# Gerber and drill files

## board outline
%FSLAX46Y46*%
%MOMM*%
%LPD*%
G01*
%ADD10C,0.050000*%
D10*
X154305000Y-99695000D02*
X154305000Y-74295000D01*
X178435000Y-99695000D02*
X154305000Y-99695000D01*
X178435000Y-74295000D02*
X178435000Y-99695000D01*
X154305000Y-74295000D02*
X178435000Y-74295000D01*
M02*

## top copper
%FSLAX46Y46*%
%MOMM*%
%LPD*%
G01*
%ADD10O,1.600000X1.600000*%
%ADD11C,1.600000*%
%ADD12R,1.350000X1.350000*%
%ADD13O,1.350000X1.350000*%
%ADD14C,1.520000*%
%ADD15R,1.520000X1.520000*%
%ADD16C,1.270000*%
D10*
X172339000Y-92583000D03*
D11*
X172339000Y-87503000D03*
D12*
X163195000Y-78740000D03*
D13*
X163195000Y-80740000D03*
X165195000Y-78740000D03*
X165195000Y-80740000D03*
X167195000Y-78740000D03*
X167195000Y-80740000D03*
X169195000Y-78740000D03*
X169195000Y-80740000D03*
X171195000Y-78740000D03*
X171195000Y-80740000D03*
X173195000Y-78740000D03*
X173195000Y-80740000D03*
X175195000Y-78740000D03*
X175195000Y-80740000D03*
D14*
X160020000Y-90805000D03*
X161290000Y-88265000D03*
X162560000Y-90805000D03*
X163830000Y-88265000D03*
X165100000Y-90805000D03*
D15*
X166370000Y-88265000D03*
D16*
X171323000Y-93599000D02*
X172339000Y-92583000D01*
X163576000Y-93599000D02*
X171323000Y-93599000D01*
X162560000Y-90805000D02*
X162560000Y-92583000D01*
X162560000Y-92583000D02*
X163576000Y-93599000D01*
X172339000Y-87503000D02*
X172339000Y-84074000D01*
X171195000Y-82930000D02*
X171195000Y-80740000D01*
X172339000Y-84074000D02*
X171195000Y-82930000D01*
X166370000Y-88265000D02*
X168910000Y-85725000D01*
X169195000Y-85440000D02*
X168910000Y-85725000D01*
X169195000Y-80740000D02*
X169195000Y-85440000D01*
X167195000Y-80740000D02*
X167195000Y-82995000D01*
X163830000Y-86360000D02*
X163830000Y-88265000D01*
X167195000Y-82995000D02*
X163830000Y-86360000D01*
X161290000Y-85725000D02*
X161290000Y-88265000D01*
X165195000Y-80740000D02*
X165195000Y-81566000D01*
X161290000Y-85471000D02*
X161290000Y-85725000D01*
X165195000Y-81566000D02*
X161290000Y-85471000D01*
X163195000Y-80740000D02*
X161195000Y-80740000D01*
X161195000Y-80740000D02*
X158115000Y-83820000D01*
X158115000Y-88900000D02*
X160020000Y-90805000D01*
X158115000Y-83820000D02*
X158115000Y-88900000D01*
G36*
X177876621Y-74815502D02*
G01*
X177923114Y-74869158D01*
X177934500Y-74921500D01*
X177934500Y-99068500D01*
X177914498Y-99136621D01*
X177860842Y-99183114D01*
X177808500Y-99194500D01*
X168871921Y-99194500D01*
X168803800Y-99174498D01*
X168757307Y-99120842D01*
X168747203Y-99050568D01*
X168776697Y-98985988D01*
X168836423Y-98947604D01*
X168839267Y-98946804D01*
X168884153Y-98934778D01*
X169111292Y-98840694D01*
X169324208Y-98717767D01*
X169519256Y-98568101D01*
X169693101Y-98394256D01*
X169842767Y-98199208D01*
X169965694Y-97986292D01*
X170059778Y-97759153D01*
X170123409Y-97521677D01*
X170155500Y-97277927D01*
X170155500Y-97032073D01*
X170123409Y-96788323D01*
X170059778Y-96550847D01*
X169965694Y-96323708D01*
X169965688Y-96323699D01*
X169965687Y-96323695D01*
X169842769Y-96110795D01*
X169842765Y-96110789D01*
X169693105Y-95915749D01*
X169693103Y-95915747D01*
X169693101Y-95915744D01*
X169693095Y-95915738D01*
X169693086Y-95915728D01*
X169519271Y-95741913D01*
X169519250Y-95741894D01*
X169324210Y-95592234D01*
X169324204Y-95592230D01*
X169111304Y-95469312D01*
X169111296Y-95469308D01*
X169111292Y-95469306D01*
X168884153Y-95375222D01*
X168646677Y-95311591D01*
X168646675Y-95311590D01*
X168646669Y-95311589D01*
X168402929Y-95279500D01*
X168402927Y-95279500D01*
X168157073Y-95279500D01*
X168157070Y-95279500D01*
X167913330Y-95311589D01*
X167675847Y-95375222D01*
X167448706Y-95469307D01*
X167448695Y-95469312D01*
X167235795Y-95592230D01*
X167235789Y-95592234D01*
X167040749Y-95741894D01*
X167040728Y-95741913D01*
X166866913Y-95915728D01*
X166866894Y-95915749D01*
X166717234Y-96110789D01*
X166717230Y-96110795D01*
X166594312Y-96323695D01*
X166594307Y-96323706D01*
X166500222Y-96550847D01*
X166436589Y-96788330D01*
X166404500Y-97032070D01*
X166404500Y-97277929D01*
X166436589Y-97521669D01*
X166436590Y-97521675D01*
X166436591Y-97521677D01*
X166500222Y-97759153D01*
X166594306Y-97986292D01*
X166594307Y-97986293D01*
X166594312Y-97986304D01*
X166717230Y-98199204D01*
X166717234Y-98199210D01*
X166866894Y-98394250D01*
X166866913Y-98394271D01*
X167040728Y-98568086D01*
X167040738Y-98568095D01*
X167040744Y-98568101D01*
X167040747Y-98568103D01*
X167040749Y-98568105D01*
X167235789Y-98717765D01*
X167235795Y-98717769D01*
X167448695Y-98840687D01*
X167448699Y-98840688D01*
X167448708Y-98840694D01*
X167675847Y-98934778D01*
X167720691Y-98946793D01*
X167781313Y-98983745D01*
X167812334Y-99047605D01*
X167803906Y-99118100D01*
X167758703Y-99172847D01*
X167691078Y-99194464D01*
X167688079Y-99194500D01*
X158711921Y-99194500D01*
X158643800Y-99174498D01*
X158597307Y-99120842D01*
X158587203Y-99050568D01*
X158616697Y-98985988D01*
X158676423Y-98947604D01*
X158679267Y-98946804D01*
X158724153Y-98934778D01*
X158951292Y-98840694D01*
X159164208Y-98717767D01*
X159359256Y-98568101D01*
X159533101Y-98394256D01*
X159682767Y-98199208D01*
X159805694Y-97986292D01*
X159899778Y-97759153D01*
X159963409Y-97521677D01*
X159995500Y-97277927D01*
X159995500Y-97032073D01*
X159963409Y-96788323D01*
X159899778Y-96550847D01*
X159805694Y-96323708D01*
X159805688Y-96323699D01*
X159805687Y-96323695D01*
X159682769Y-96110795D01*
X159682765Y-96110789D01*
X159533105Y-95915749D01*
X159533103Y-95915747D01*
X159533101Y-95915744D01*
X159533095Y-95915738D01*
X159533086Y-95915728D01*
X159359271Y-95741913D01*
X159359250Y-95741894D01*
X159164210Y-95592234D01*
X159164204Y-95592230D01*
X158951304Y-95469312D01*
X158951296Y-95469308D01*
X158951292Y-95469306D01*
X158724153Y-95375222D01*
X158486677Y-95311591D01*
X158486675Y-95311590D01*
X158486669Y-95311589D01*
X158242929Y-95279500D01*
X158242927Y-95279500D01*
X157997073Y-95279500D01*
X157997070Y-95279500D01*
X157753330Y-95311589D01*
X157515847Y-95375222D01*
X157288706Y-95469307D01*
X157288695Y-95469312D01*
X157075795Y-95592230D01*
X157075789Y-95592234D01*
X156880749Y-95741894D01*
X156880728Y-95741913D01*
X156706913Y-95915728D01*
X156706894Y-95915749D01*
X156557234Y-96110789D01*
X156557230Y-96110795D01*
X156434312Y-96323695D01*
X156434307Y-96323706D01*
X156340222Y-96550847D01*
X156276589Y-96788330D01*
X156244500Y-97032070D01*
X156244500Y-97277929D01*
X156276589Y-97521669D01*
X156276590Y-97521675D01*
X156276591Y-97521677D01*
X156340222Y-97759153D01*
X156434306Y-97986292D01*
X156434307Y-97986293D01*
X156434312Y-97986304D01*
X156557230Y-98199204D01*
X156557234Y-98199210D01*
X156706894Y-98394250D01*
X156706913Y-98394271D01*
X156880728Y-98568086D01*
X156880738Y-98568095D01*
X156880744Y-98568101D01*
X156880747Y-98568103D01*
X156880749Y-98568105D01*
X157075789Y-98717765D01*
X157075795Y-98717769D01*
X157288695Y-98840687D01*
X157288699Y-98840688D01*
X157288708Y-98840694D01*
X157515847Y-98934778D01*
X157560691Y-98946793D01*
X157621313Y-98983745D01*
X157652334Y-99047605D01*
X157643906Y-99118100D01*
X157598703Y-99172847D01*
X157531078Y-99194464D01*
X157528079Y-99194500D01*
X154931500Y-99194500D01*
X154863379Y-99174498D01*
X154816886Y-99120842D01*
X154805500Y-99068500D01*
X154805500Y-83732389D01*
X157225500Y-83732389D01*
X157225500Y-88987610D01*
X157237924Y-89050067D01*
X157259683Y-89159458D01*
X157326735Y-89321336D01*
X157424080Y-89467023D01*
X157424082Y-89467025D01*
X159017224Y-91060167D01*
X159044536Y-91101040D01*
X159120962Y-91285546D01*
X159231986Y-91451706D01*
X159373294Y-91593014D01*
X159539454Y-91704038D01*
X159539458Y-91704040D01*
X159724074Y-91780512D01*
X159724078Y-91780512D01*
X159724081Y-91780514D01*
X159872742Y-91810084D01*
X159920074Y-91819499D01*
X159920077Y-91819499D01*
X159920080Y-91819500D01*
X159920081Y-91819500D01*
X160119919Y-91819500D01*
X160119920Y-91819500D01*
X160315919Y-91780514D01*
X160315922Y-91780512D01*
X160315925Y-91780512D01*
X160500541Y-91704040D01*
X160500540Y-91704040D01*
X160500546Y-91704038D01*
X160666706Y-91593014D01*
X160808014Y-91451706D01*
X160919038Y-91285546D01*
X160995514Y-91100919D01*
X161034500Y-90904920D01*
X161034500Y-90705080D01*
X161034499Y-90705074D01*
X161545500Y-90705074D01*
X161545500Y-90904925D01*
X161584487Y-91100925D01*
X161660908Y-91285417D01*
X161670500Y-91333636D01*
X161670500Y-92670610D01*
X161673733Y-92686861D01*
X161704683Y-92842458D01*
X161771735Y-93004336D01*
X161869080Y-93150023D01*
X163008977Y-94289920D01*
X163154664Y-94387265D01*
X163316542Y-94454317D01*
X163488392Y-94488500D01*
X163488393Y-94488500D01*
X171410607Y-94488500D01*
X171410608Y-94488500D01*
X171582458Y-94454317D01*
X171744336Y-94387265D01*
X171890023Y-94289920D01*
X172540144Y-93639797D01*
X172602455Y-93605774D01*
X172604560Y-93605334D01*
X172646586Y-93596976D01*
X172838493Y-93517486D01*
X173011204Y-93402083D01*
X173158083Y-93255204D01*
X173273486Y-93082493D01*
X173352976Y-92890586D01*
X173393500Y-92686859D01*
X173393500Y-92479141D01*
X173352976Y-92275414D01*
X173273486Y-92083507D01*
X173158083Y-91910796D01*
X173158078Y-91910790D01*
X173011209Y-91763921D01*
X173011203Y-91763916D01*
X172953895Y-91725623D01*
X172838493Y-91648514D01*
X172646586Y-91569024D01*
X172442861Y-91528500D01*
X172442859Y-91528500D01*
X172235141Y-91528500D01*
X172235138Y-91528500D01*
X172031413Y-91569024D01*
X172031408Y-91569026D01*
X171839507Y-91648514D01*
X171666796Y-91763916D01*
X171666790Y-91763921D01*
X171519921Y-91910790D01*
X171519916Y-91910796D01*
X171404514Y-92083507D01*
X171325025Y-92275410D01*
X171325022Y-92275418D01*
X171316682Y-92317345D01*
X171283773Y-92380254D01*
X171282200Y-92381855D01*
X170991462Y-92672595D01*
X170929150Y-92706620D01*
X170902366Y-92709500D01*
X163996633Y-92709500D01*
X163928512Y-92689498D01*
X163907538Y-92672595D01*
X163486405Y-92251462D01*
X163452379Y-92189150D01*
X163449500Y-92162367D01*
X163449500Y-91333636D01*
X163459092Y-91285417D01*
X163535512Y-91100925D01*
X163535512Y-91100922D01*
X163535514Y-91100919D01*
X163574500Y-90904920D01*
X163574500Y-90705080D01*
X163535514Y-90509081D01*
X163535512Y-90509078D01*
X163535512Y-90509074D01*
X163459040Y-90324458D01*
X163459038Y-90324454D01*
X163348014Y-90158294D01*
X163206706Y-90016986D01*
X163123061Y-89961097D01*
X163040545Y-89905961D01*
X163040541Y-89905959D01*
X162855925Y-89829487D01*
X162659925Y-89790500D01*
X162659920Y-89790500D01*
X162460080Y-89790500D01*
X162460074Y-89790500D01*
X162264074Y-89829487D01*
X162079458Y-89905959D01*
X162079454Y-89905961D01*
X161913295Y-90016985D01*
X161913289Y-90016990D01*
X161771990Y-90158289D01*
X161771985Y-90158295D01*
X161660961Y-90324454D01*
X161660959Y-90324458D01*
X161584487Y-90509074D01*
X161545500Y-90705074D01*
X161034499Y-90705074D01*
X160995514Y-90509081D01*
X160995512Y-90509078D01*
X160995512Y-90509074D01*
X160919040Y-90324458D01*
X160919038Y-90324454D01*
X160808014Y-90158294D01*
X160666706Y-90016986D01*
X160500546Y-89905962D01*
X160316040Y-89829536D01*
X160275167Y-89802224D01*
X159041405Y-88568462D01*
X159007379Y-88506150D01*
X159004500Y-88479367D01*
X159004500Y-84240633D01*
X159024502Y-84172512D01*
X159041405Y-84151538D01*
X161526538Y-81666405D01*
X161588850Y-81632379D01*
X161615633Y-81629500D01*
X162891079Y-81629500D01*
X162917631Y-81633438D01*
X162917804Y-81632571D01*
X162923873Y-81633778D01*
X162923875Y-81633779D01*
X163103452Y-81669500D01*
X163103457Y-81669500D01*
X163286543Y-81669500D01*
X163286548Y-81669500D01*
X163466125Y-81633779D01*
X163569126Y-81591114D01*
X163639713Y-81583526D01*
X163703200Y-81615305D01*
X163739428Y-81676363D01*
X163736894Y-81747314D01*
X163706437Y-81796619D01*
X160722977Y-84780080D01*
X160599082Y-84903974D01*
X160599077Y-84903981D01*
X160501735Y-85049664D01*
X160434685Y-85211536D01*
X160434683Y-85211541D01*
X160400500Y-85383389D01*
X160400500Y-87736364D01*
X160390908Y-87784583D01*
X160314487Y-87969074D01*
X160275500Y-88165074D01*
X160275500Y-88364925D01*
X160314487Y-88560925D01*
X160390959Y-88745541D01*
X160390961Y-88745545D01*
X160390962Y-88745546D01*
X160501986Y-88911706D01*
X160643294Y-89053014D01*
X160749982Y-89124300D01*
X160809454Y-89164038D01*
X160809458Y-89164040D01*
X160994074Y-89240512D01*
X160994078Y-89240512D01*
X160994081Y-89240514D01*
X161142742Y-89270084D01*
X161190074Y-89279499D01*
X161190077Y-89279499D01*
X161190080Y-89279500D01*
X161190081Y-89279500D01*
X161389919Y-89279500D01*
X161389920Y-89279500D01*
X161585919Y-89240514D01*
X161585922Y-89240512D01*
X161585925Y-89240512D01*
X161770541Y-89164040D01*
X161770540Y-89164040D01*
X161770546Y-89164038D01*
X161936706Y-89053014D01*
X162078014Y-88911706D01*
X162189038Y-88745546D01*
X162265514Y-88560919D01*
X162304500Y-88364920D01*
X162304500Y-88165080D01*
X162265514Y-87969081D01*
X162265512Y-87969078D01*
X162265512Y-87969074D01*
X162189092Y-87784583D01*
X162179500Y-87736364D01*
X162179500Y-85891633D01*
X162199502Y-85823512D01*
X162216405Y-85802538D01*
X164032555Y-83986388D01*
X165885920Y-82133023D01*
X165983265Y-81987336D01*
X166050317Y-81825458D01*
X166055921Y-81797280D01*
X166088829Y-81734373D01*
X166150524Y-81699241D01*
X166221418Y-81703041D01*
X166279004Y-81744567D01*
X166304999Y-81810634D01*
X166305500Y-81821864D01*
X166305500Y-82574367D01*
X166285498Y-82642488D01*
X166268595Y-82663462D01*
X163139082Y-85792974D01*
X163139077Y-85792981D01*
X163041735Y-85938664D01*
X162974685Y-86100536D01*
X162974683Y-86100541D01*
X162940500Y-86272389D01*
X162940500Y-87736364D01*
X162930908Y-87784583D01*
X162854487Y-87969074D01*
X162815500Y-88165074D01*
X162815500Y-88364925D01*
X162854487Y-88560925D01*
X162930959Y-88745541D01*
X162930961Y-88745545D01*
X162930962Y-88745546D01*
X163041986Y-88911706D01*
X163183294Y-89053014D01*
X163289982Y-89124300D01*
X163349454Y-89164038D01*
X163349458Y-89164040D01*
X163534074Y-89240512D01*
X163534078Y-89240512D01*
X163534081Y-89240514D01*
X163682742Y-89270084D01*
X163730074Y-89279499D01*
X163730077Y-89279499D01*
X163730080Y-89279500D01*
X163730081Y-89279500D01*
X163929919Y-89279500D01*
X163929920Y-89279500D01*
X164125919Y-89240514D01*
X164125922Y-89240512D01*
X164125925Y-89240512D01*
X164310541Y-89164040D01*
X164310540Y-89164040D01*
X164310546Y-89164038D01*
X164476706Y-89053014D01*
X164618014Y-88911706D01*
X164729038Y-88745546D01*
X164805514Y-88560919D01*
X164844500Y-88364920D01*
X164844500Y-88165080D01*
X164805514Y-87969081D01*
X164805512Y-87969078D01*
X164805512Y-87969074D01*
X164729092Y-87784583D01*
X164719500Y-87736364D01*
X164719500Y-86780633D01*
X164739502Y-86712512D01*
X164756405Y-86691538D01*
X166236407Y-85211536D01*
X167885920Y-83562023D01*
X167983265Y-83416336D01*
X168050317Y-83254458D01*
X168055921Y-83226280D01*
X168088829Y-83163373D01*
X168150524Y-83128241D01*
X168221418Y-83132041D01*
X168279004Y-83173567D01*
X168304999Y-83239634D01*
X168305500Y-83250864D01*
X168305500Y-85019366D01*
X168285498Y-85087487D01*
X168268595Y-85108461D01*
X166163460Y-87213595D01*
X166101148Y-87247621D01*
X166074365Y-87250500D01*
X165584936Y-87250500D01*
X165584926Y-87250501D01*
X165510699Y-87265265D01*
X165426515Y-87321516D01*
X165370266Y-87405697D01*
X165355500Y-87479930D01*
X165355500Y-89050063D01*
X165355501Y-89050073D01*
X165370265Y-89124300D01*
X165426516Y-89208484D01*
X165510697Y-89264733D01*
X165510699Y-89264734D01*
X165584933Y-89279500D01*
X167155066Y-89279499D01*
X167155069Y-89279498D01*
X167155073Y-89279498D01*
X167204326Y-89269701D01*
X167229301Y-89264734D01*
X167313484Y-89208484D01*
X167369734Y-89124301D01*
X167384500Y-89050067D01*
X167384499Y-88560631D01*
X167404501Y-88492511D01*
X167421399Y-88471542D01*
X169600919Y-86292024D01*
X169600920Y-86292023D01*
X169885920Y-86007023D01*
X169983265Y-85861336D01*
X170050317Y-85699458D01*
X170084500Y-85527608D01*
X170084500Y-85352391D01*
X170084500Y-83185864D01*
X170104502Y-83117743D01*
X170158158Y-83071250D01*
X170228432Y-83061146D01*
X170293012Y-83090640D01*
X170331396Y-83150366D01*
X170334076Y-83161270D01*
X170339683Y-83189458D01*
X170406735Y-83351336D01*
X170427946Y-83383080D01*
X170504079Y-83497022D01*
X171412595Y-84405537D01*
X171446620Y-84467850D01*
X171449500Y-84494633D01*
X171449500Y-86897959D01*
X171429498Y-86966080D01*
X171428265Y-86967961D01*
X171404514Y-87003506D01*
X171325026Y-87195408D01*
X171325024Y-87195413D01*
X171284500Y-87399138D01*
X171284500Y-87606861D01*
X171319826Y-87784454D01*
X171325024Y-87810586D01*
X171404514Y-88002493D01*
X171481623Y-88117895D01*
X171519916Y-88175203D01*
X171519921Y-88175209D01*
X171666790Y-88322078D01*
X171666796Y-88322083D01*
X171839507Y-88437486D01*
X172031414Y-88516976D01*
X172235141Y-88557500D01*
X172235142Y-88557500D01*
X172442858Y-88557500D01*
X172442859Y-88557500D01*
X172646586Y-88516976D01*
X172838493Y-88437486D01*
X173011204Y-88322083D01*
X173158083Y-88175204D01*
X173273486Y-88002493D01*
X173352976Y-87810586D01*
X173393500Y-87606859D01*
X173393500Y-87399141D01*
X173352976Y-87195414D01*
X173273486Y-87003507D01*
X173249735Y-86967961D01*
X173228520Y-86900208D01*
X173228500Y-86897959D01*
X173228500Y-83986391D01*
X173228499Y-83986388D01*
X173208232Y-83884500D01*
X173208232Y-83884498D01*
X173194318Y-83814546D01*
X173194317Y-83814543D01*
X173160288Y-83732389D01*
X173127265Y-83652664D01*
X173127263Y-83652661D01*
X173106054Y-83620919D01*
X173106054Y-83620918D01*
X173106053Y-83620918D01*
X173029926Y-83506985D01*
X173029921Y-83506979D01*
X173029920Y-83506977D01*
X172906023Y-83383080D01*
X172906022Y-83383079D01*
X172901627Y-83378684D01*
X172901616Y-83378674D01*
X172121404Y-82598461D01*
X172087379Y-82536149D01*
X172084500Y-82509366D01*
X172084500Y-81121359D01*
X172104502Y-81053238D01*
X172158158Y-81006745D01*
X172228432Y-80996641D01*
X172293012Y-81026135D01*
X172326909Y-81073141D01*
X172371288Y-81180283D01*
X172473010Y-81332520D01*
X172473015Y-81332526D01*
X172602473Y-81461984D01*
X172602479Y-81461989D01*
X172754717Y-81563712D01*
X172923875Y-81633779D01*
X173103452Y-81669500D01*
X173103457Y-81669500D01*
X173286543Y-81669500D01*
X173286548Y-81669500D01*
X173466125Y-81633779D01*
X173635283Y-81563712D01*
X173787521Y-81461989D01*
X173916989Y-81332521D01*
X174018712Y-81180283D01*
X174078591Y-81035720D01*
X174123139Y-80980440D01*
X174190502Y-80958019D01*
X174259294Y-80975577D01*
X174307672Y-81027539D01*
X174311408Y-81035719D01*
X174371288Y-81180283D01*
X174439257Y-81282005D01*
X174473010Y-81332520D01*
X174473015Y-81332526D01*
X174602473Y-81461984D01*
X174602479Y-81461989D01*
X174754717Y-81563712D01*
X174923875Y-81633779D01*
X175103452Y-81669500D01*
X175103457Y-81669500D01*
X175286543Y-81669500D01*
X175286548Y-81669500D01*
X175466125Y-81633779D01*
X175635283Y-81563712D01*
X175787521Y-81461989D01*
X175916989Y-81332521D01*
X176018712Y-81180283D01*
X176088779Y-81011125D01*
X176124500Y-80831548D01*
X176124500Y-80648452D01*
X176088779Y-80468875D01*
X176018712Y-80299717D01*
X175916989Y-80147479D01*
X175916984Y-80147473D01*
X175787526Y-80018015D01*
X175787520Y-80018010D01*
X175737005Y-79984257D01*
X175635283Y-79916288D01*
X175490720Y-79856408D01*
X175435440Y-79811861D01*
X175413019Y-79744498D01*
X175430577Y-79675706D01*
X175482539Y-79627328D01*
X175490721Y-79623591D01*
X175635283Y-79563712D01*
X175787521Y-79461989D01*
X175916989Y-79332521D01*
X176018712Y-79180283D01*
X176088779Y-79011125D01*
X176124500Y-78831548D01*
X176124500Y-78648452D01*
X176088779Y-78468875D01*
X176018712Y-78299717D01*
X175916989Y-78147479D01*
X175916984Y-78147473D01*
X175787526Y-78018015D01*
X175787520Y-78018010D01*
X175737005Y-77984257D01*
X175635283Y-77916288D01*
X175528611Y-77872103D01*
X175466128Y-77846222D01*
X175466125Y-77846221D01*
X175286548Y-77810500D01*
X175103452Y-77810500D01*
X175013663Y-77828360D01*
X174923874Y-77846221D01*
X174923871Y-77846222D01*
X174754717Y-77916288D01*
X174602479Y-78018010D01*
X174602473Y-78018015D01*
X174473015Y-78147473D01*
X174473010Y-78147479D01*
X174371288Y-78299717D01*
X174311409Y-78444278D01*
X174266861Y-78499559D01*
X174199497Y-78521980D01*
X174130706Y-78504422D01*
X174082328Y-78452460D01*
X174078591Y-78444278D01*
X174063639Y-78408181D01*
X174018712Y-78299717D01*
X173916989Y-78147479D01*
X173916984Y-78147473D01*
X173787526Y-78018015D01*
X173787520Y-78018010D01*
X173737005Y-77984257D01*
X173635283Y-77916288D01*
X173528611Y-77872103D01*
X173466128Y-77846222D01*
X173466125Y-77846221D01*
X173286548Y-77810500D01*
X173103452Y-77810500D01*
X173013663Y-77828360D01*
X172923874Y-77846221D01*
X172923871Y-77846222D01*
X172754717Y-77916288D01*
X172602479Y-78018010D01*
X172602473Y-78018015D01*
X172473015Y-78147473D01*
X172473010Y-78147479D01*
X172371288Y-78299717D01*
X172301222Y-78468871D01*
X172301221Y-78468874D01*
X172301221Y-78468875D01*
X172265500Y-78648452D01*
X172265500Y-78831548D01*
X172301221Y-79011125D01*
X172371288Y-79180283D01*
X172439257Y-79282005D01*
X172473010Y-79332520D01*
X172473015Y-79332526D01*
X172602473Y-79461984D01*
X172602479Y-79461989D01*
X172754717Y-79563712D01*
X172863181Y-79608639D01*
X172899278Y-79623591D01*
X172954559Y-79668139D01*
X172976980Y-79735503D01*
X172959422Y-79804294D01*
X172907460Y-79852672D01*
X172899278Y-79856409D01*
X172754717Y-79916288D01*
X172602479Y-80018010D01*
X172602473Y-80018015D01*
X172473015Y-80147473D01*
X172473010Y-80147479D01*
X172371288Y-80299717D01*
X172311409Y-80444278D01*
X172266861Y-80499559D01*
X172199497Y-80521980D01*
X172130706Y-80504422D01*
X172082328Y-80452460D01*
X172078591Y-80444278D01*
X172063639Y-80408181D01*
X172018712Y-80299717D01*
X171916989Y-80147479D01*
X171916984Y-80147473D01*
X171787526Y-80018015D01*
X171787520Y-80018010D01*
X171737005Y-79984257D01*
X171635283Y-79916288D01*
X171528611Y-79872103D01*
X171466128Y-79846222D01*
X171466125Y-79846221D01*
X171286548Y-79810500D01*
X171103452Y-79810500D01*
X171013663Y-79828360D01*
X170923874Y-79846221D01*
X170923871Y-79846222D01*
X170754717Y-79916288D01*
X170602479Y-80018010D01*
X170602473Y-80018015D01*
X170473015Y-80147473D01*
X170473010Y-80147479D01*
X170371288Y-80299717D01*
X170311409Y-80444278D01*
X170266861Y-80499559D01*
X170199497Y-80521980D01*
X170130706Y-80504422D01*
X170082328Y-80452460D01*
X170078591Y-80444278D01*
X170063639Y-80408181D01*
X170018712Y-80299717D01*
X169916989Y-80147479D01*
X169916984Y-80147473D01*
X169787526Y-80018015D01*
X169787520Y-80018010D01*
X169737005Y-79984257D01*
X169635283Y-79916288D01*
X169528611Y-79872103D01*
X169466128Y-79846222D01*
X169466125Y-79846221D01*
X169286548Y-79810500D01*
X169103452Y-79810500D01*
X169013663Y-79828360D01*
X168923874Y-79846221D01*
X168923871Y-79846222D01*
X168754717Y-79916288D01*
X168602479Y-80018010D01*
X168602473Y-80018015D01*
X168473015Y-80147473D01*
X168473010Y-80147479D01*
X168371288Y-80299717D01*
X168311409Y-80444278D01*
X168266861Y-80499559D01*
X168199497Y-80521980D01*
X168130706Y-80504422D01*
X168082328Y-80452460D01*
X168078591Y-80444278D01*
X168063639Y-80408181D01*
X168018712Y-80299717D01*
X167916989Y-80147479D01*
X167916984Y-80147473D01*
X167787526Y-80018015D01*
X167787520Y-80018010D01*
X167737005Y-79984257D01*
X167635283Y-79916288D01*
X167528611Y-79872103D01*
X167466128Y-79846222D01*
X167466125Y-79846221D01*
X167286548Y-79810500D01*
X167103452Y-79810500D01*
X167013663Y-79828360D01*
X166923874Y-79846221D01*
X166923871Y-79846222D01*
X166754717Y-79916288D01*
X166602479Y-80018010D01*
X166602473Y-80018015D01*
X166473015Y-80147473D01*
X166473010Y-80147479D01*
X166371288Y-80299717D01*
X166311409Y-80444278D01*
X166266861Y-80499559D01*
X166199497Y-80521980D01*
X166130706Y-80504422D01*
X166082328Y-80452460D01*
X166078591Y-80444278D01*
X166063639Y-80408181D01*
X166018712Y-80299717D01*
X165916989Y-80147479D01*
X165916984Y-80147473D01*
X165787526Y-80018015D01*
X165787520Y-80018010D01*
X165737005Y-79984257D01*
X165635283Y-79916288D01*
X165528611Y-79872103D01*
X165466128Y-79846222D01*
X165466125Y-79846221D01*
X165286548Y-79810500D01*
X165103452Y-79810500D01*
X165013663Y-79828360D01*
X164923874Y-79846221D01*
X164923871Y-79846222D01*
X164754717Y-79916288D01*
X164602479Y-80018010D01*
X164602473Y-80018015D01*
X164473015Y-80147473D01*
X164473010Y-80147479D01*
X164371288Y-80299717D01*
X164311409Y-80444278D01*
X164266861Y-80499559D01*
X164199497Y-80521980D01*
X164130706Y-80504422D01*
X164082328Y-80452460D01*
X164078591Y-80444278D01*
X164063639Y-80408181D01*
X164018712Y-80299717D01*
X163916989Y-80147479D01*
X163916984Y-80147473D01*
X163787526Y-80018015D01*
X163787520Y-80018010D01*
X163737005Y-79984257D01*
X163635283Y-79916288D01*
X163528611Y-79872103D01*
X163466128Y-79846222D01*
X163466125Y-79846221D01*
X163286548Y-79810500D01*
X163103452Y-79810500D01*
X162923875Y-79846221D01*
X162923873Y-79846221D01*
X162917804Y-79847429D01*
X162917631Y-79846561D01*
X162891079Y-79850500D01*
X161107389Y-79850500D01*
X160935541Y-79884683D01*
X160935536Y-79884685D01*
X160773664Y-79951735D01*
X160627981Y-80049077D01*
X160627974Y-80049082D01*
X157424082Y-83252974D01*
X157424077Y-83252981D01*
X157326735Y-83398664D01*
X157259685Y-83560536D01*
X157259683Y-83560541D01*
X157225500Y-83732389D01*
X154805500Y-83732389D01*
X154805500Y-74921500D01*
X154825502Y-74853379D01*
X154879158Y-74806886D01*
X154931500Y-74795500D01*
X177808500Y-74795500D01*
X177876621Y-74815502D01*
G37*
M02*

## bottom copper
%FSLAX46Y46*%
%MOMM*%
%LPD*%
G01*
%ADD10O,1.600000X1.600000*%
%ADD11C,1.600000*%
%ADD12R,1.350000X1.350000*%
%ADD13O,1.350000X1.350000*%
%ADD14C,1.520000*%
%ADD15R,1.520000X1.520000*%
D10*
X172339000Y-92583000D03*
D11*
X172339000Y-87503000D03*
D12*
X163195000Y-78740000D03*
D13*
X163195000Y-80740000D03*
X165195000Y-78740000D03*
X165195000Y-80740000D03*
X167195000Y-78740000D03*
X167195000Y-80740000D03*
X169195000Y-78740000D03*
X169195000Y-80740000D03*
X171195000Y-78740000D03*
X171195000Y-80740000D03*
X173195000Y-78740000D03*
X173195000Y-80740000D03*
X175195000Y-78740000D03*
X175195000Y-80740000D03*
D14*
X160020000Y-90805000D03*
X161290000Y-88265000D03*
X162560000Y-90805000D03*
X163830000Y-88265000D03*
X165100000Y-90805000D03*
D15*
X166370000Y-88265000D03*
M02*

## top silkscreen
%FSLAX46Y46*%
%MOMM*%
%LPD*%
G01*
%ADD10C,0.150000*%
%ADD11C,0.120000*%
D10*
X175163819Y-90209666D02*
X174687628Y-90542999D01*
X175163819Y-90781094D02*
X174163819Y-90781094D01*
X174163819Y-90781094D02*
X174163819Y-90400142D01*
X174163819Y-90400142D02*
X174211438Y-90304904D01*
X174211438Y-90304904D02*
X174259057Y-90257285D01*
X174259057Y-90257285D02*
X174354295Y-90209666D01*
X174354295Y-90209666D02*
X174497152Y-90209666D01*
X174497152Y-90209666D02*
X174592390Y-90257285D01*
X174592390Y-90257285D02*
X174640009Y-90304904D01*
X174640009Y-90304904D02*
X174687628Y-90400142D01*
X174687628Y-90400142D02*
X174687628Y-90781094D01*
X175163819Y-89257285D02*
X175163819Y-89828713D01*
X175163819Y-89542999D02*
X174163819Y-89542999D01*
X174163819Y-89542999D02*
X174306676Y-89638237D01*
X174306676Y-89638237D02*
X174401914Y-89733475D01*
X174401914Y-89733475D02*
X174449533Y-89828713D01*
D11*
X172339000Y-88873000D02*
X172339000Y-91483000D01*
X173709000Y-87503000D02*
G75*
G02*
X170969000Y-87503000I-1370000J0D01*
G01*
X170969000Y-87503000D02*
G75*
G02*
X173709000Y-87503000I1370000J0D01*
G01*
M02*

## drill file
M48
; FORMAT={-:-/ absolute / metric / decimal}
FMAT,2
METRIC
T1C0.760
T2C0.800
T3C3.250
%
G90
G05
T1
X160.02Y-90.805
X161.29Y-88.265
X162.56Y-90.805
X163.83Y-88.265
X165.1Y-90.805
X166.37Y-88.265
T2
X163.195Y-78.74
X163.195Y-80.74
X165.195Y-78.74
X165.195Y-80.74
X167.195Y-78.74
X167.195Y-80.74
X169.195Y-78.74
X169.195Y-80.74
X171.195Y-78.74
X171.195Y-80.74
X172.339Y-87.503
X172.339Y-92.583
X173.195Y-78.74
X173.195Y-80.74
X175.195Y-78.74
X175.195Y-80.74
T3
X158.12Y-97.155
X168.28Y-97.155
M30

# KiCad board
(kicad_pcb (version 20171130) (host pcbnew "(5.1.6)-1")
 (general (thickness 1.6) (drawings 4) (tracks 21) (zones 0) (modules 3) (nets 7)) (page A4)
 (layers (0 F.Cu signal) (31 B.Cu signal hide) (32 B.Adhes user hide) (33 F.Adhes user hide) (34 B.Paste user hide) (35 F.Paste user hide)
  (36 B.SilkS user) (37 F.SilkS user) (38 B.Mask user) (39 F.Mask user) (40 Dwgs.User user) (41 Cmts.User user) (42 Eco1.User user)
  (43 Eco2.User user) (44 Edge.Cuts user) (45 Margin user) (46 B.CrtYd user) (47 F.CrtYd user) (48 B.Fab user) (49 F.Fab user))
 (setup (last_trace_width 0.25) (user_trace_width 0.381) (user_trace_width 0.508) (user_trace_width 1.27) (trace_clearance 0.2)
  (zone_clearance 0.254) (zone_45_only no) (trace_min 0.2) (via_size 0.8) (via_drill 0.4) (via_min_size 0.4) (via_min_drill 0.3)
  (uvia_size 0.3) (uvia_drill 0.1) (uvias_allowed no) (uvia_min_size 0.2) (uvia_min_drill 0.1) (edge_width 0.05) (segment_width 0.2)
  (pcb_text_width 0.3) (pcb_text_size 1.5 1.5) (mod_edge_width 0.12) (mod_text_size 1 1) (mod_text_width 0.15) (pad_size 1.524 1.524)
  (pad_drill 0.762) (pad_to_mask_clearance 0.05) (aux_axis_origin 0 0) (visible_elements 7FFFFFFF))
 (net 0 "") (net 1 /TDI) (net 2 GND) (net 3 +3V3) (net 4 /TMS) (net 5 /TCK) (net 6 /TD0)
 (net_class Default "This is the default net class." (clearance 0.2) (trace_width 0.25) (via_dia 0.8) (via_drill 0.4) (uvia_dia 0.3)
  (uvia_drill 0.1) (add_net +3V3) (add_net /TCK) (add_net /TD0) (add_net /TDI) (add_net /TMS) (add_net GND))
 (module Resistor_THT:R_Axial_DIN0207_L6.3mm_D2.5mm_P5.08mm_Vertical (layer F.Cu) (at 172.339 87.503 270)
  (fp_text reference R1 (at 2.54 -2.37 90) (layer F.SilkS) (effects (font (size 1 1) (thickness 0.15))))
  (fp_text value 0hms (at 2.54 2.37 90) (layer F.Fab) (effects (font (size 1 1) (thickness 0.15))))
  (fp_line (start 1.37 0) (end 3.98 0) (layer F.SilkS) (width 0.12))
  (fp_circle (center 0 0) (end 1.37 0) (layer F.SilkS) (width 0.12))
  (pad 2 thru_hole oval (at 5.08 0 270) (size 1.6 1.6) (drill 0.8) (layers *.Cu *.Mask) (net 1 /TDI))
  (pad 1 thru_hole circle (at 0 0 270) (size 1.6 1.6) (drill 0.8) (layers *.Cu *.Mask) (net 1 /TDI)))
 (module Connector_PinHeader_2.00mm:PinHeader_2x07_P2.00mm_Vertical (layer B.Cu) (at 163.195 78.74 270)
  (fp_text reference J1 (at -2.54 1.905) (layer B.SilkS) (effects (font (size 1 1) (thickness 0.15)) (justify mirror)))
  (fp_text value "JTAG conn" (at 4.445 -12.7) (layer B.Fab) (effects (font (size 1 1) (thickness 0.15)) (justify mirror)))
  (pad 1 thru_hole rect (at 0 0 270) (size 1.35 1.35) (drill 0.8) (layers *.Cu *.Mask) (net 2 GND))
  (pad 14 thru_hole oval (at 2 0 270) (size 1.35 1.35) (drill 0.8) (layers *.Cu *.Mask) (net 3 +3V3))
  (pad 2 thru_hole oval (at 0 -2 270) (size 1.35 1.35) (drill 0.8) (layers *.Cu *.Mask) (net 2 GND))
  (pad 13 thru_hole oval (at 2 -2 270) (size 1.35 1.35) (drill 0.8) (layers *.Cu *.Mask) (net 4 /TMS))
  (pad 3 thru_hole oval (at 0 -4 270) (size 1.35 1.35) (drill 0.8) (layers *.Cu *.Mask) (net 2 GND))
  (pad 12 thru_hole oval (at 2 -4 270) (size 1.35 1.35) (drill 0.8) (layers *.Cu *.Mask) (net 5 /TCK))
  (pad 4 thru_hole oval (at 0 -6 270) (size 1.35 1.35) (drill 0.8) (layers *.Cu *.Mask) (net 2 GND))
  (pad 11 thru_hole oval (at 2 -6 270) (size 1.35 1.35) (drill 0.8) (layers *.Cu *.Mask) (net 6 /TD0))
  (pad 5 thru_hole oval (at 0 -8 270) (size 1.35 1.35) (drill 0.8) (layers *.Cu *.Mask) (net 2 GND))
  (pad 10 thru_hole oval (at 2 -8 270) (size 1.35 1.35) (drill 0.8) (layers *.Cu *.Mask) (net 1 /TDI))
  (pad 6 thru_hole oval (at 0 -10 270) (size 1.35 1.35) (drill 0.8) (layers *.Cu *.Mask))
  (pad 9 thru_hole oval (at 2 -10 270) (size 1.35 1.35) (drill 0.8) (layers *.Cu *.Mask))
  (pad 7 thru_hole oval (at 0 -12 270) (size 1.35 1.35) (drill 0.8) (layers *.Cu *.Mask))
  (pad 8 thru_hole oval (at 2 -12 270) (size 1.35 1.35) (drill 0.8) (layers *.Cu *.Mask)))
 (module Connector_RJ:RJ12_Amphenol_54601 (layer B.Cu) (at 166.37 88.265 180)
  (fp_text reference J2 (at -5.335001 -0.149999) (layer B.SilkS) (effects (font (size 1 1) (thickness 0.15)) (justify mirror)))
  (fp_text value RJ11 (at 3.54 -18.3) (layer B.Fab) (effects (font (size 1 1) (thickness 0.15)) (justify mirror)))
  (pad "" np_thru_hole circle (at 8.25 -8.89 180) (size 3.25 3.25) (drill 3.25) (layers *.Cu *.Mask))
  (pad 6 thru_hole circle (at 6.35 -2.54 180) (size 1.52 1.52) (drill 0.76) (layers *.Cu *.Mask) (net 3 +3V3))
  (pad 5 thru_hole circle (at 5.08 0 180) (size 1.52 1.52) (drill 0.76) (layers *.Cu *.Mask) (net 4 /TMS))
  (pad 4 thru_hole circle (at 3.81 -2.54 180) (size 1.52 1.52) (drill 0.76) (layers *.Cu *.Mask) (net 1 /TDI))
  (pad 3 thru_hole circle (at 2.54 0 180) (size 1.52 1.52) (drill 0.76) (layers *.Cu *.Mask) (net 5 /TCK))
  (pad 2 thru_hole circle (at 1.27 -2.54 180) (size 1.52 1.52) (drill 0.76) (layers *.Cu *.Mask) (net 2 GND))
  (pad "" np_thru_hole circle (at -1.91 -8.89 180) (size 3.25 3.25) (drill 3.25) (layers *.Cu *.Mask))
  (pad 1 thru_hole rect (at 0 0 180) (size 1.52 1.52) (drill 0.76) (layers *.Cu *.Mask) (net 6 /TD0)))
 (gr_line (start 154.305 99.695) (end 154.305 74.295) (layer Edge.Cuts) (width 0.05))
 (gr_line (start 178.435 99.695) (end 154.305 99.695) (layer Edge.Cuts) (width 0.05))
 (gr_line (start 178.435 74.295) (end 178.435 99.695) (layer Edge.Cuts) (width 0.05))
 (gr_line (start 154.305 74.295) (end 178.435 74.295) (layer Edge.Cuts) (width 0.05))
 (segment (start 171.323 93.599) (end 172.339 92.583) (width 1.27) (layer F.Cu) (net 1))
 (segment (start 163.576 93.599) (end 171.323 93.599) (width 1.27) (layer F.Cu) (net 1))
 (segment (start 162.56 90.805) (end 162.56 92.583) (width 1.27) (layer F.Cu) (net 1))
 (segment (start 162.56 92.583) (end 163.576 93.599) (width 1.27) (layer F.Cu) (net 1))
 (segment (start 172.339 87.503) (end 172.339 84.074) (width 1.27) (layer F.Cu) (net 1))
 (segment (start 171.195 82.93) (end 171.195 80.74) (width 1.27) (layer F.Cu) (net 1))
 (segment (start 172.339 84.074) (end 171.195 82.93) (width 1.27) (layer F.Cu) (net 1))
 (segment (start 166.37 88.265) (end 168.91 85.725) (width 1.27) (layer F.Cu) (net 6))
 (segment (start 169.195 85.44) (end 168.91 85.725) (width 1.27) (layer F.Cu) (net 6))
 (segment (start 169.195 80.74) (end 169.195 85.44) (width 1.27) (layer F.Cu) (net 6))
 (segment (start 167.195 80.74) (end 167.195 82.995) (width 1.27) (layer F.Cu) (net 5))
 (segment (start 163.83 86.36) (end 163.83 88.265) (width 1.27) (layer F.Cu) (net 5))
 (segment (start 167.195 82.995) (end 163.83 86.36) (width 1.27) (layer F.Cu) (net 5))
 (segment (start 161.29 85.725) (end 161.29 88.265) (width 1.27) (layer F.Cu) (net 4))
 (segment (start 165.195 80.74) (end 165.195 81.566) (width 1.27) (layer F.Cu) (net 4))
 (segment (start 161.29 85.471) (end 161.29 85.725) (width 1.27) (layer F.Cu) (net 4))
 (segment (start 165.195 81.566) (end 161.29 85.471) (width 1.27) (layer F.Cu) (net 4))
 (segment (start 163.195 80.74) (end 161.195 80.74) (width 1.27) (layer F.Cu) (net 3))
 (segment (start 161.195 80.74) (end 158.115 83.82) (width 1.27) (layer F.Cu) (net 3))
 (segment (start 158.115 88.9) (end 160.02 90.805) (width 1.27) (layer F.Cu) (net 3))
 (segment (start 158.115 83.82) (end 158.115 88.9) (width 1.27) (layer F.Cu) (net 3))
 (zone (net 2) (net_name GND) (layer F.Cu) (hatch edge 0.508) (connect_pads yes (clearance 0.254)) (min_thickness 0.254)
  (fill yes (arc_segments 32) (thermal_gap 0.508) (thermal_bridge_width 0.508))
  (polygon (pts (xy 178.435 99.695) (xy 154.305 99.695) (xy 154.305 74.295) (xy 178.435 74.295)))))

